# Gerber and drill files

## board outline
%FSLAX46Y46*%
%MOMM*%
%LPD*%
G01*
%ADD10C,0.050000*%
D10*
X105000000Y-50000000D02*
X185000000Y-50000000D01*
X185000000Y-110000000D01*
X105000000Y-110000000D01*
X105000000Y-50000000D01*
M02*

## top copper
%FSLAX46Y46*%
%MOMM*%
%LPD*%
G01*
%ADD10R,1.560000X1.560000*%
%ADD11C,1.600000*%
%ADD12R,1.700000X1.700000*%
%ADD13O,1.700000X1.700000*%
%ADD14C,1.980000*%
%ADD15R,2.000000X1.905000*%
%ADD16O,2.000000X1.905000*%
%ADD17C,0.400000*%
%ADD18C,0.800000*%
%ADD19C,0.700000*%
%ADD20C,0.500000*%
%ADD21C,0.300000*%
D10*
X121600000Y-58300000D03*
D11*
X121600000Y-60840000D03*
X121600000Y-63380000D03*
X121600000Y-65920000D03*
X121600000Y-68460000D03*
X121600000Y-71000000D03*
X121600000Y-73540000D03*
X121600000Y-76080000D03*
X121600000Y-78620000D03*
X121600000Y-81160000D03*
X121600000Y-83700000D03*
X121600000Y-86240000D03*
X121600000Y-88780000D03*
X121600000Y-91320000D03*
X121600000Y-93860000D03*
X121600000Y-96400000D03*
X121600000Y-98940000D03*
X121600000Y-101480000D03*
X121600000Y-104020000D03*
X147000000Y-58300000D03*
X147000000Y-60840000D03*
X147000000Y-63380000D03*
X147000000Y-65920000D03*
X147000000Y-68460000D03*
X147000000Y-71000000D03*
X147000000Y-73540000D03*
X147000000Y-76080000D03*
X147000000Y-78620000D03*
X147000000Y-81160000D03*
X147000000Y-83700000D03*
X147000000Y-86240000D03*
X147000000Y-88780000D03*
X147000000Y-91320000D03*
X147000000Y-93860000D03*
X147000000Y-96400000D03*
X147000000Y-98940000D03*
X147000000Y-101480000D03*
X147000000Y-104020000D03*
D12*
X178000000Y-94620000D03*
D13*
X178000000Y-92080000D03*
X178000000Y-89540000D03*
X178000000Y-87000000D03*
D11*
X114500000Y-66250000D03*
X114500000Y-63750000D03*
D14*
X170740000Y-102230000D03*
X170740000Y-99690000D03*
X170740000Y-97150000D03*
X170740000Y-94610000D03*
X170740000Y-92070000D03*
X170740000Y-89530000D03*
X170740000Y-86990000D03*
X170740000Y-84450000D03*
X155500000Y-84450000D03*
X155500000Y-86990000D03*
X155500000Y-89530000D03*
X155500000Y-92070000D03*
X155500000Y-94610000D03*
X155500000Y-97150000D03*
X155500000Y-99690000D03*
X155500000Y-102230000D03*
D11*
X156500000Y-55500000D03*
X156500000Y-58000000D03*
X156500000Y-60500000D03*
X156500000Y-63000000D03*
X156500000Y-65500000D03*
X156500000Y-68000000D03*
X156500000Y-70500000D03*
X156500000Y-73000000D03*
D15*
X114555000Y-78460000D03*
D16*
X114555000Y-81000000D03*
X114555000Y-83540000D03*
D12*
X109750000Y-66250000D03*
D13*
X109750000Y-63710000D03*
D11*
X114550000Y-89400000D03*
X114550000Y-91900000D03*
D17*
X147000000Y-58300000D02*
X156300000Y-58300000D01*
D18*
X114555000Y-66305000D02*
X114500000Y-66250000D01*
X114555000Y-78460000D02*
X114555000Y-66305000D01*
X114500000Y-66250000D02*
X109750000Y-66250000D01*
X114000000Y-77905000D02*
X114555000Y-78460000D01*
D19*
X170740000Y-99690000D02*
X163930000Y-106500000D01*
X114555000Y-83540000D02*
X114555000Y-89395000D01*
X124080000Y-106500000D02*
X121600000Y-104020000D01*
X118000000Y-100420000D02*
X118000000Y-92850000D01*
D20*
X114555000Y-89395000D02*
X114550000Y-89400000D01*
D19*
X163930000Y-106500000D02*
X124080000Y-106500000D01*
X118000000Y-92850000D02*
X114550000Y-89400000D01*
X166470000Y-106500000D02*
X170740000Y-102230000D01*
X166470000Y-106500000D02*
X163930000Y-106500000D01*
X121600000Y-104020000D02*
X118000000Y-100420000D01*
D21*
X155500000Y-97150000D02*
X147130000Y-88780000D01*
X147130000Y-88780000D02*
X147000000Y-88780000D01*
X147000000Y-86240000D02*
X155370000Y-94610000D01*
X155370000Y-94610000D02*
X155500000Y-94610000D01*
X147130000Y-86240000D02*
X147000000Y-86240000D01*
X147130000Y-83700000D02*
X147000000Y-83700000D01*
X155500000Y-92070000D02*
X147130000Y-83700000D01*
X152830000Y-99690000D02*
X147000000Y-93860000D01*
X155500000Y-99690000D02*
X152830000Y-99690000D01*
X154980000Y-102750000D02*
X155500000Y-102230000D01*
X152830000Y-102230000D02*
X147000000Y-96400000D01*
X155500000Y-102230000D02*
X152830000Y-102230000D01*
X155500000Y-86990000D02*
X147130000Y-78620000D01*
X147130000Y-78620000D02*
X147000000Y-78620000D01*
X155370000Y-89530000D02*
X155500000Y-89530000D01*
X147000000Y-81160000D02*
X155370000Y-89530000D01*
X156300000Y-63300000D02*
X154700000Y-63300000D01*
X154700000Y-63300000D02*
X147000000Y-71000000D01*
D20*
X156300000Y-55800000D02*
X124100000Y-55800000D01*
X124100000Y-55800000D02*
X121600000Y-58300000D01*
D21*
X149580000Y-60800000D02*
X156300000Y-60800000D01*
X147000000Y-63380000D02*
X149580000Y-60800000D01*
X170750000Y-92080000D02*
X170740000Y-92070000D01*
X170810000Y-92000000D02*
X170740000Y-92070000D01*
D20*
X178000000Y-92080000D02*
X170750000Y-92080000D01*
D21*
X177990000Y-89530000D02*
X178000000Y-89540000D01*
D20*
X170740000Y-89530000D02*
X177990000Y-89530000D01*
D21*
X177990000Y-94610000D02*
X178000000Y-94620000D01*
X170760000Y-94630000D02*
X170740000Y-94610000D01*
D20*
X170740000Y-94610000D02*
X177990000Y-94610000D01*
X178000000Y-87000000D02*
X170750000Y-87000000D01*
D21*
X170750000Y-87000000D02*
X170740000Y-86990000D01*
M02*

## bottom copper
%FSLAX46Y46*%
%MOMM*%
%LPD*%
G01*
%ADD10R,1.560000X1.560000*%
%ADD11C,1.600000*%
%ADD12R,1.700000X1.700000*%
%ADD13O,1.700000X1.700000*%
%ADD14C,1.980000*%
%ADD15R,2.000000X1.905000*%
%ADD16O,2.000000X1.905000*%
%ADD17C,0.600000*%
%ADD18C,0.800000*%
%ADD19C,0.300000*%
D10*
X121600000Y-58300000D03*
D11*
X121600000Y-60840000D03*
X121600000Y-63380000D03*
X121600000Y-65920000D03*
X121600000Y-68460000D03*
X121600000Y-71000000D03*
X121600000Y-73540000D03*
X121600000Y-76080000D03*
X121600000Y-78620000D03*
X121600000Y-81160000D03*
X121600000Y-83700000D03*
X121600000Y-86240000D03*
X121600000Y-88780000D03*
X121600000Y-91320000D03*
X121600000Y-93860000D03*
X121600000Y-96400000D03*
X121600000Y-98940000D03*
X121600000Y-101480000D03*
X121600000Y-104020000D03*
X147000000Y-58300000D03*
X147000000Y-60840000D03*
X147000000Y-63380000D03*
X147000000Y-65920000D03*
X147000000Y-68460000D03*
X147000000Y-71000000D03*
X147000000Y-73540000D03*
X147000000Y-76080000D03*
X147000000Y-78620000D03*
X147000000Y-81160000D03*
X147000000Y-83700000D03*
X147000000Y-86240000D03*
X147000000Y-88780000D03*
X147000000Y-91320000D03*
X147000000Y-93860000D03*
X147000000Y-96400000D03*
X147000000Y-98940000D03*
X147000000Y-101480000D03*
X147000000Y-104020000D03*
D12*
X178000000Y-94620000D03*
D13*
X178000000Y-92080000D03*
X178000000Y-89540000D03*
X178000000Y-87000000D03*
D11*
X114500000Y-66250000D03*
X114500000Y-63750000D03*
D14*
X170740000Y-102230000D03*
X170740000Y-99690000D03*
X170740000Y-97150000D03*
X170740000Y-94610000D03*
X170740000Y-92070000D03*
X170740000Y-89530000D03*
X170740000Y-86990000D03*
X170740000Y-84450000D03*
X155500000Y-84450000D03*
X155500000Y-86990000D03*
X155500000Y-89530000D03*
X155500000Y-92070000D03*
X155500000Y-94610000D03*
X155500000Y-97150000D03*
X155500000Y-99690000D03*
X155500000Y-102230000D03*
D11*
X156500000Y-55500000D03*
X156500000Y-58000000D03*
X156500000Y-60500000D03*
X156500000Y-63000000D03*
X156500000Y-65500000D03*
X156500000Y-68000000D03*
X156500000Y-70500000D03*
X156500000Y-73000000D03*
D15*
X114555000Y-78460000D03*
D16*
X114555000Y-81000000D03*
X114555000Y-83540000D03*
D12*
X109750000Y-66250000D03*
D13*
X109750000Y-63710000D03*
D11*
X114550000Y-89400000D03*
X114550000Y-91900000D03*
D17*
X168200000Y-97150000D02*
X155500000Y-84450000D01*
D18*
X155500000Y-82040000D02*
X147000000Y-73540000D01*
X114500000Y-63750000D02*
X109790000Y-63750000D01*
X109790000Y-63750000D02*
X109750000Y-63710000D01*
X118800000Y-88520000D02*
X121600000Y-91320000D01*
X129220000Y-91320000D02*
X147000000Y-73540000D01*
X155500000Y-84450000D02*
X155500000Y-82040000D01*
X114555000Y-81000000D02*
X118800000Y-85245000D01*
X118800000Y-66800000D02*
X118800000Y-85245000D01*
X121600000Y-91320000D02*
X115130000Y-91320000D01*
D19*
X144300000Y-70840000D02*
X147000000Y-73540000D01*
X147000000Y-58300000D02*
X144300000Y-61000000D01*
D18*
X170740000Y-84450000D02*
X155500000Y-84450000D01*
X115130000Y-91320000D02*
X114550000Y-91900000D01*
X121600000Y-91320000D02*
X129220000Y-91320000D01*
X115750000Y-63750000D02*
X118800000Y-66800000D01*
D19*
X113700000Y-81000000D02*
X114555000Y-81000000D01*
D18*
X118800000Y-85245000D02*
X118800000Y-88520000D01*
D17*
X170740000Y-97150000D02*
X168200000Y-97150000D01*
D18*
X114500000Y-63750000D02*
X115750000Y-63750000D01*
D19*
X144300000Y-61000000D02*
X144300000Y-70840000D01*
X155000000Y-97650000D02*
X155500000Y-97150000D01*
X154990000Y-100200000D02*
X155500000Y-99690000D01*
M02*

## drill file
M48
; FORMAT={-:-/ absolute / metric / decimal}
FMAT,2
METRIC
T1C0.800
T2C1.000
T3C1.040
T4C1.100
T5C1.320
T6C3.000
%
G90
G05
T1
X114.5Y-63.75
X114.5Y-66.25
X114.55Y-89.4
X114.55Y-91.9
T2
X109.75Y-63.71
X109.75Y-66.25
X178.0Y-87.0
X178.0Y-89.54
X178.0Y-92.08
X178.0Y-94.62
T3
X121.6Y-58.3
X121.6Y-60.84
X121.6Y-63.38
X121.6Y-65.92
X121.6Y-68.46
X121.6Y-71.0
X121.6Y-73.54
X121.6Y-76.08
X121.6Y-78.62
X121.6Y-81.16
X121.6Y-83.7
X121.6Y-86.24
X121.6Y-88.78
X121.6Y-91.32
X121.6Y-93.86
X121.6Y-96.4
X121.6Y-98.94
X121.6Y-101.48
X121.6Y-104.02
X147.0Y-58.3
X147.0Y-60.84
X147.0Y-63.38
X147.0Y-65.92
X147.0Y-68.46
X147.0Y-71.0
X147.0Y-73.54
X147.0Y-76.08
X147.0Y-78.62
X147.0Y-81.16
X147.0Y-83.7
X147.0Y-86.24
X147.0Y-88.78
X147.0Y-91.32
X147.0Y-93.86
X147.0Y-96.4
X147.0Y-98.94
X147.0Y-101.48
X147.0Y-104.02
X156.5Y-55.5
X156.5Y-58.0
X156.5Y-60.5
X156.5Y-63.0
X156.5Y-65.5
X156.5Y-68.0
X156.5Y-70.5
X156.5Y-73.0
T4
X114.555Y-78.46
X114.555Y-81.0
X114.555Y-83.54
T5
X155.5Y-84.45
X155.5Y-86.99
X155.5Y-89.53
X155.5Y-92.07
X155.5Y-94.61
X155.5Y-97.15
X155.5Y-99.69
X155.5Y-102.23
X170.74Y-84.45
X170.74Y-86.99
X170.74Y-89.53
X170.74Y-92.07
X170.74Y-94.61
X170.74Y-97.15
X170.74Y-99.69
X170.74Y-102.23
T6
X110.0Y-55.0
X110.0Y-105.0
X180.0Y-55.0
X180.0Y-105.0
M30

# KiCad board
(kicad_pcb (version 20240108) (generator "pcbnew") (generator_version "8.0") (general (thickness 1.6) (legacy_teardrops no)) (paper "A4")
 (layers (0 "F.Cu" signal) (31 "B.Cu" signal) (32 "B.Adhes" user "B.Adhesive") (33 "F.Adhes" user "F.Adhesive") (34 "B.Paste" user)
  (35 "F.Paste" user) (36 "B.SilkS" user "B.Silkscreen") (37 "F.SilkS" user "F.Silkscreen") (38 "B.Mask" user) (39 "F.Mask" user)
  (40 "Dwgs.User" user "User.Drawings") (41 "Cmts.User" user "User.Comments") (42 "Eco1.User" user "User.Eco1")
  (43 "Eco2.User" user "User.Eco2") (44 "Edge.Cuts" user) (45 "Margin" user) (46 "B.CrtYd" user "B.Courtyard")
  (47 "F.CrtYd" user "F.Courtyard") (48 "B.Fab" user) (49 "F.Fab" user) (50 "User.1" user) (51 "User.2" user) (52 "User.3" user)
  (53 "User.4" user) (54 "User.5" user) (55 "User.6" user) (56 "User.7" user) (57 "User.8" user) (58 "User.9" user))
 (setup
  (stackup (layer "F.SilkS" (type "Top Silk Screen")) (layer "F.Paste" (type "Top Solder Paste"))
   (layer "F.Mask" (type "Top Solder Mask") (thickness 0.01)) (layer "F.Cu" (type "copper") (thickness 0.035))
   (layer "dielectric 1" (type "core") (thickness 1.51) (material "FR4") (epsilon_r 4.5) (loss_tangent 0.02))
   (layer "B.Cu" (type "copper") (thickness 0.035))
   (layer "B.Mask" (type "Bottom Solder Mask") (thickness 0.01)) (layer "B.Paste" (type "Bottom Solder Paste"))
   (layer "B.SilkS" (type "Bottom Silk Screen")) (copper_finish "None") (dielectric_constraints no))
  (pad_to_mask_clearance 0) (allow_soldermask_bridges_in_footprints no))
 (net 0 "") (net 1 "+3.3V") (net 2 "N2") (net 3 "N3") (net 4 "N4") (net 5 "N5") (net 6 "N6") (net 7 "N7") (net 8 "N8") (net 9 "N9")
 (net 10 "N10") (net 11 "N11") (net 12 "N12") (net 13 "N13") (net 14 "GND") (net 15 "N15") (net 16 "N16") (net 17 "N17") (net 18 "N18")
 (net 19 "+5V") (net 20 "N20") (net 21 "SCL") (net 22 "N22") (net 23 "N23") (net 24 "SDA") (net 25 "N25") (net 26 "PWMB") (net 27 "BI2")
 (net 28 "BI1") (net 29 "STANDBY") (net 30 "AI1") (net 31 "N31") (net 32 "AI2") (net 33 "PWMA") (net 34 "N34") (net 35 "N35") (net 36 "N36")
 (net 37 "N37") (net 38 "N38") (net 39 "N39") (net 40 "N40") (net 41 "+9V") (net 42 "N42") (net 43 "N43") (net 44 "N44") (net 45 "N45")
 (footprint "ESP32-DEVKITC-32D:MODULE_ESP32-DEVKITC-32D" (layer "F.Cu") (at 134.3 78.06)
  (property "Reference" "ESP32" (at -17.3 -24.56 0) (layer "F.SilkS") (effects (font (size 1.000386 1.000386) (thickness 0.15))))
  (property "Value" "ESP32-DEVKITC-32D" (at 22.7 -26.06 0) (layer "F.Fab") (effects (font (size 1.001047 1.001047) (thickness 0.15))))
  (pad "J2-1" thru_hole rect (at -12.7 -19.76) (size 1.56 1.56) (drill 1.04) (layers "*.Cu" "*.Mask") (remove_unused_layers no)
   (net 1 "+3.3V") (solder_mask_margin 0.102))
  (pad "J2-2" thru_hole circle (at -12.7 -17.22) (size 1.6 1.6) (drill 1.04) (layers "*.Cu" "*.Mask") (remove_unused_layers no) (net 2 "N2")
   (solder_mask_margin 0.102))
  (pad "J2-3" thru_hole circle (at -12.7 -14.68) (size 1.6 1.6) (drill 1.04) (layers "*.Cu" "*.Mask") (remove_unused_layers no) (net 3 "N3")
   (solder_mask_margin 0.102))
  (pad "J2-4" thru_hole circle (at -12.7 -12.14) (size 1.6 1.6) (drill 1.04) (layers "*.Cu" "*.Mask") (remove_unused_layers no) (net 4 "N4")
   (solder_mask_margin 0.102))
  (pad "J2-5" thru_hole circle (at -12.7 -9.6) (size 1.6 1.6) (drill 1.04) (layers "*.Cu" "*.Mask") (remove_unused_layers no) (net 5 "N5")
   (solder_mask_margin 0.102))
  (pad "J2-6" thru_hole circle (at -12.7 -7.06) (size 1.6 1.6) (drill 1.04) (layers "*.Cu" "*.Mask") (remove_unused_layers no) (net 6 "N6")
   (solder_mask_margin 0.102))
  (pad "J2-7" thru_hole circle (at -12.7 -4.52) (size 1.6 1.6) (drill 1.04) (layers "*.Cu" "*.Mask") (remove_unused_layers no) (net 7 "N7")
   (solder_mask_margin 0.102))
  (pad "J2-8" thru_hole circle (at -12.7 -1.98) (size 1.6 1.6) (drill 1.04) (layers "*.Cu" "*.Mask") (remove_unused_layers no) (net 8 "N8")
   (solder_mask_margin 0.102))
  (pad "J2-9" thru_hole circle (at -12.7 0.56) (size 1.6 1.6) (drill 1.04) (layers "*.Cu" "*.Mask") (remove_unused_layers no) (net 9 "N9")
   (solder_mask_margin 0.102))
  (pad "J2-10" thru_hole circle (at -12.7 3.1) (size 1.6 1.6) (drill 1.04) (layers "*.Cu" "*.Mask") (remove_unused_layers no) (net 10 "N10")
   (solder_mask_margin 0.102))
  (pad "J2-11" thru_hole circle (at -12.7 5.64) (size 1.6 1.6) (drill 1.04) (layers "*.Cu" "*.Mask") (remove_unused_layers no)
   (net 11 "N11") (solder_mask_margin 0.102))
  (pad "J2-12" thru_hole circle (at -12.7 8.18) (size 1.6 1.6) (drill 1.04) (layers "*.Cu" "*.Mask") (remove_unused_layers no)
   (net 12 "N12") (solder_mask_margin 0.102))
  (pad "J2-13" thru_hole circle (at -12.7 10.72) (size 1.6 1.6) (drill 1.04) (layers "*.Cu" "*.Mask") (remove_unused_layers no)
   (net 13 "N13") (solder_mask_margin 0.102))
  (pad "J2-14" thru_hole circle (at -12.7 13.26) (size 1.6 1.6) (drill 1.04) (layers "*.Cu" "*.Mask") (remove_unused_layers no)
   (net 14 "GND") (solder_mask_margin 0.102))
  (pad "J2-15" thru_hole circle (at -12.7 15.8) (size 1.6 1.6) (drill 1.04) (layers "*.Cu" "*.Mask") (remove_unused_layers no)
   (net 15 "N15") (solder_mask_margin 0.102))
  (pad "J2-16" thru_hole circle (at -12.7 18.34) (size 1.6 1.6) (drill 1.04) (layers "*.Cu" "*.Mask") (remove_unused_layers no)
   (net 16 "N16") (solder_mask_margin 0.102))
  (pad "J2-17" thru_hole circle (at -12.7 20.88) (size 1.6 1.6) (drill 1.04) (layers "*.Cu" "*.Mask") (remove_unused_layers no)
   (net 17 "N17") (solder_mask_margin 0.102))
  (pad "J2-18" thru_hole circle (at -12.7 23.42) (size 1.6 1.6) (drill 1.04) (layers "*.Cu" "*.Mask") (remove_unused_layers no)
   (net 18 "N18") (solder_mask_margin 0.102))
  (pad "J2-19" thru_hole circle (at -12.7 25.96) (size 1.6 1.6) (drill 1.04) (layers "*.Cu" "*.Mask") (remove_unused_layers no)
   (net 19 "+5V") (solder_mask_margin 0.102))
  (pad "J3-1" thru_hole circle (at 12.7 -19.76) (size 1.6 1.6) (drill 1.04) (layers "*.Cu" "*.Mask") (remove_unused_layers no)
   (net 14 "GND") (solder_mask_margin 0.102))
  (pad "J3-2" thru_hole circle (at 12.7 -17.22) (size 1.6 1.6) (drill 1.04) (layers "*.Cu" "*.Mask") (remove_unused_layers no)
   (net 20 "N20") (solder_mask_margin 0.102))
  (pad "J3-3" thru_hole circle (at 12.7 -14.68) (size 1.6 1.6) (drill 1.04) (layers "*.Cu" "*.Mask") (remove_unused_layers no)
   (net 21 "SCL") (solder_mask_margin 0.102))
  (pad "J3-4" thru_hole circle (at 12.7 -12.14) (size 1.6 1.6) (drill 1.04) (layers "*.Cu" "*.Mask") (remove_unused_layers no)
   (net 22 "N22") (solder_mask_margin 0.102))
  (pad "J3-5" thru_hole circle (at 12.7 -9.6) (size 1.6 1.6) (drill 1.04) (layers "*.Cu" "*.Mask") (remove_unused_layers no) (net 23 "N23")
   (solder_mask_margin 0.102))
  (pad "J3-6" thru_hole circle (at 12.7 -7.06) (size 1.6 1.6) (drill 1.04) (layers "*.Cu" "*.Mask") (remove_unused_layers no) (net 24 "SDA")
   (solder_mask_margin 0.102))
  (pad "J3-7" thru_hole circle (at 12.7 -4.52) (size 1.6 1.6) (drill 1.04) (layers "*.Cu" "*.Mask") (remove_unused_layers no) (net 14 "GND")
   (solder_mask_margin 0.102))
  (pad "J3-8" thru_hole circle (at 12.7 -1.98) (size 1.6 1.6) (drill 1.04) (layers "*.Cu" "*.Mask") (remove_unused_layers no) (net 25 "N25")
   (solder_mask_margin 0.102))
  (pad "J3-9" thru_hole circle (at 12.7 0.56) (size 1.6 1.6) (drill 1.04) (layers "*.Cu" "*.Mask") (remove_unused_layers no) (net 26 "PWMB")
   (solder_mask_margin 0.102))
  (pad "J3-10" thru_hole circle (at 12.7 3.1) (size 1.6 1.6) (drill 1.04) (layers "*.Cu" "*.Mask") (remove_unused_layers no) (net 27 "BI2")
   (solder_mask_margin 0.102))
  (pad "J3-11" thru_hole circle (at 12.7 5.64) (size 1.6 1.6) (drill 1.04) (layers "*.Cu" "*.Mask") (remove_unused_layers no) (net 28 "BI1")
   (solder_mask_margin 0.102))
  (pad "J3-12" thru_hole circle (at 12.7 8.18) (size 1.6 1.6) (drill 1.04) (layers "*.Cu" "*.Mask") (remove_unused_layers no)
   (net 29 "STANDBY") (solder_mask_margin 0.102))
  (pad "J3-13" thru_hole circle (at 12.7 10.72) (size 1.6 1.6) (drill 1.04) (layers "*.Cu" "*.Mask") (remove_unused_layers no)
   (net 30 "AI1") (solder_mask_margin 0.102))
  (pad "J3-14" thru_hole circle (at 12.7 13.26) (size 1.6 1.6) (drill 1.04) (layers "*.Cu" "*.Mask") (remove_unused_layers no)
   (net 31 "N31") (solder_mask_margin 0.102))
  (pad "J3-15" thru_hole circle (at 12.7 15.8) (size 1.6 1.6) (drill 1.04) (layers "*.Cu" "*.Mask") (remove_unused_layers no) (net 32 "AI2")
   (solder_mask_margin 0.102))
  (pad "J3-16" thru_hole circle (at 12.7 18.34) (size 1.6 1.6) (drill 1.04) (layers "*.Cu" "*.Mask") (remove_unused_layers no)
   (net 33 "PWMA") (solder_mask_margin 0.102))
  (pad "J3-17" thru_hole circle (at 12.7 20.88) (size 1.6 1.6) (drill 1.04) (layers "*.Cu" "*.Mask") (remove_unused_layers no)
   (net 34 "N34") (solder_mask_margin 0.102))
  (pad "J3-18" thru_hole circle (at 12.7 23.42) (size 1.6 1.6) (drill 1.04) (layers "*.Cu" "*.Mask") (remove_unused_layers no)
   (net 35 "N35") (solder_mask_margin 0.102))
  (pad "J3-19" thru_hole circle (at 12.7 25.96) (size 1.6 1.6) (drill 1.04) (layers "*.Cu" "*.Mask") (remove_unused_layers no)
   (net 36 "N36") (solder_mask_margin 0.102)))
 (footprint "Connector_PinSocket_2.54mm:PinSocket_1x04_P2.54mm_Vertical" (layer "F.Cu") (at 178 94.62 180)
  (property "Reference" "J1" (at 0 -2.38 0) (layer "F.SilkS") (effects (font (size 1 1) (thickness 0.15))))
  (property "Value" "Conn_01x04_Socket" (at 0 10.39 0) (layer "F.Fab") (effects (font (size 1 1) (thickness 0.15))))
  (pad "1" thru_hole rect (at 0 0 180) (size 1.7 1.7) (drill 1) (layers "*.Cu" "*.Mask") (remove_unused_layers no) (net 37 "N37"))
  (pad "2" thru_hole oval (at 0 2.54 180) (size 1.7 1.7) (drill 1) (layers "*.Cu" "*.Mask") (remove_unused_layers no) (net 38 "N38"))
  (pad "3" thru_hole oval (at 0 5.08 180) (size 1.7 1.7) (drill 1) (layers "*.Cu" "*.Mask") (remove_unused_layers no) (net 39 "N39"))
  (pad "4" thru_hole oval (at 0 7.62 180) (size 1.7 1.7) (drill 1) (layers "*.Cu" "*.Mask") (remove_unused_layers no) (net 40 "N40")))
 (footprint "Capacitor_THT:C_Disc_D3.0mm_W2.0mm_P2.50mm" (layer "F.Cu") (at 114.5 66.25 90)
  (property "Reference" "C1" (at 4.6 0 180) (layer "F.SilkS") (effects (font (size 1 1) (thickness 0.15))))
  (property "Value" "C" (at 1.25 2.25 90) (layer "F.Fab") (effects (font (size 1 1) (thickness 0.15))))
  (pad "1" thru_hole circle (at 0 0 90) (size 1.6 1.6) (drill 0.8) (layers "*.Cu" "*.Mask") (remove_unused_layers no) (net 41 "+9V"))
  (pad "2" thru_hole circle (at 2.5 0 90) (size 1.6 1.6) (drill 0.8) (layers "*.Cu" "*.Mask") (remove_unused_layers no) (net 14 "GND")))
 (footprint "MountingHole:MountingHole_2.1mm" (layer "F.Cu") (at 180 55)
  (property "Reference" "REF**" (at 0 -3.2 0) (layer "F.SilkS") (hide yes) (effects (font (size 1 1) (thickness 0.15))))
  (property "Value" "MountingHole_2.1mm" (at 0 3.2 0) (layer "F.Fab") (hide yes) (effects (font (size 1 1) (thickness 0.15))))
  (pad "" np_thru_hole circle (at 0 0) (size 3 3) (drill 3) (layers "F&B.Cu" "*.Mask")))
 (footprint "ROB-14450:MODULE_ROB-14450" (layer "F.Cu") (at 163.12 93.34 180)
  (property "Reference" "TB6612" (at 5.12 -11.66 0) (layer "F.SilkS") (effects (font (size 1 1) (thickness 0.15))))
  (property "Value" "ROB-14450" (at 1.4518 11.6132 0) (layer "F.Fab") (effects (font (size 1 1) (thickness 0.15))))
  (pad "1" thru_hole circle (at -7.62 -8.89 180) (size 1.98 1.98) (drill 1.32) (layers "*.Cu" "*.Mask") (remove_unused_layers no)
   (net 19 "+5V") (solder_mask_margin 0.102))
  (pad "2" thru_hole circle (at -7.62 -6.35 180) (size 1.98 1.98) (drill 1.32) (layers "*.Cu" "*.Mask") (remove_unused_layers no)
   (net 19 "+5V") (solder_mask_margin 0.102))
  (pad "3" thru_hole circle (at -7.62 -3.81 180) (size 1.98 1.98) (drill 1.32) (layers "*.Cu" "*.Mask") (remove_unused_layers no)
   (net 14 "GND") (solder_mask_margin 0.102))
  (pad "4" thru_hole circle (at -7.62 -1.27 180) (size 1.98 1.98) (drill 1.32) (layers "*.Cu" "*.Mask") (remove_unused_layers no)
   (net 37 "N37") (solder_mask_margin 0.102))
  (pad "5" thru_hole circle (at -7.62 1.27 180) (size 1.98 1.98) (drill 1.32) (layers "*.Cu" "*.Mask") (remove_unused_layers no)
   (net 38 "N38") (solder_mask_margin 0.102))
  (pad "6" thru_hole circle (at -7.62 3.81 180) (size 1.98 1.98) (drill 1.32) (layers "*.Cu" "*.Mask") (remove_unused_layers no)
   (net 39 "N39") (solder_mask_margin 0.102))
  (pad "7" thru_hole circle (at -7.62 6.35 180) (size 1.98 1.98) (drill 1.32) (layers "*.Cu" "*.Mask") (remove_unused_layers no)
   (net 40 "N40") (solder_mask_margin 0.102))
  (pad "8" thru_hole circle (at -7.62 8.89 180) (size 1.98 1.98) (drill 1.32) (layers "*.Cu" "*.Mask") (remove_unused_layers no)
   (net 14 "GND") (solder_mask_margin 0.102))
  (pad "9" thru_hole circle (at 7.62 8.89 180) (size 1.98 1.98) (drill 1.32) (layers "*.Cu" "*.Mask") (remove_unused_layers no)
   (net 14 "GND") (solder_mask_margin 0.102))
  (pad "10" thru_hole circle (at 7.62 6.35 180) (size 1.98 1.98) (drill 1.32) (layers "*.Cu" "*.Mask") (remove_unused_layers no)
   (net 26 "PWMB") (solder_mask_margin 0.102))
  (pad "11" thru_hole circle (at 7.62 3.81 180) (size 1.98 1.98) (drill 1.32) (layers "*.Cu" "*.Mask") (remove_unused_layers no)
   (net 27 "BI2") (solder_mask_margin 0.102))
  (pad "12" thru_hole circle (at 7.62 1.27 180) (size 1.98 1.98) (drill 1.32) (layers "*.Cu" "*.Mask") (remove_unused_layers no)
   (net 28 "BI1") (solder_mask_margin 0.102))
  (pad "13" thru_hole circle (at 7.62 -1.27 180) (size 1.98 1.98) (drill 1.32) (layers "*.Cu" "*.Mask") (remove_unused_layers no)
   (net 29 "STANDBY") (solder_mask_margin 0.102))
  (pad "14" thru_hole circle (at 7.62 -3.81 180) (size 1.98 1.98) (drill 1.32) (layers "*.Cu" "*.Mask") (remove_unused_layers no)
   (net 30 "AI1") (solder_mask_margin 0.102))
  (pad "15" thru_hole circle (at 7.62 -6.35 180) (size 1.98 1.98) (drill 1.32) (layers "*.Cu" "*.Mask") (remove_unused_layers no)
   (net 32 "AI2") (solder_mask_margin 0.102))
  (pad "16" thru_hole circle (at 7.62 -8.89 180) (size 1.98 1.98) (drill 1.32) (layers "*.Cu" "*.Mask") (remove_unused_layers no)
   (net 33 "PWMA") (solder_mask_margin 0.102)))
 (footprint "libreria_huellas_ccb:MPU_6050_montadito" (layer "F.Cu") (at 155 75.2)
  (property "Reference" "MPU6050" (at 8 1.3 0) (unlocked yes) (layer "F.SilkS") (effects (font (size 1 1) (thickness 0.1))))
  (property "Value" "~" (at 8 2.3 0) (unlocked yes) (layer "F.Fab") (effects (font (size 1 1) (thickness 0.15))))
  (pad "1" thru_hole circle (at 1.5 -19.7) (size 1.6 1.6) (drill 1.04) (layers "*.Cu" "*.Mask") (remove_unused_layers no) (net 1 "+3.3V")
   (solder_mask_margin 0.102))
  (pad "2" thru_hole circle (at 1.5 -17.2) (size 1.6 1.6) (drill 1.04) (layers "*.Cu" "*.Mask") (remove_unused_layers no) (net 14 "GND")
   (solder_mask_margin 0.102))
  (pad "3" thru_hole circle (at 1.5 -14.7) (size 1.6 1.6) (drill 1.04) (layers "*.Cu" "*.Mask") (remove_unused_layers no) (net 21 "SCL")
   (solder_mask_margin 0.102))
  (pad "4" thru_hole circle (at 1.5 -12.2) (size 1.6 1.6) (drill 1.04) (layers "*.Cu" "*.Mask") (remove_unused_layers no) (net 24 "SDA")
   (solder_mask_margin 0.102))
  (pad "5" thru_hole circle (at 1.5 -9.7) (size 1.6 1.6) (drill 1.04) (layers "*.Cu" "*.Mask") (remove_unused_layers no) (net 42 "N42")
   (solder_mask_margin 0.102))
  (pad "6" thru_hole circle (at 1.5 -7.2) (size 1.6 1.6) (drill 1.04) (layers "*.Cu" "*.Mask") (remove_unused_layers no) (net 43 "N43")
   (solder_mask_margin 0.102))
  (pad "7" thru_hole circle (at 1.5 -4.7) (size 1.6 1.6) (drill 1.04) (layers "*.Cu" "*.Mask") (remove_unused_layers no) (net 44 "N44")
   (solder_mask_margin 0.102))
  (pad "8" thru_hole circle (at 1.5 -2.2) (size 1.6 1.6) (drill 1.04) (layers "*.Cu" "*.Mask") (remove_unused_layers no) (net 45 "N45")
   (solder_mask_margin 0.102)))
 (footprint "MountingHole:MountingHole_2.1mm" (layer "F.Cu") (at 110 55)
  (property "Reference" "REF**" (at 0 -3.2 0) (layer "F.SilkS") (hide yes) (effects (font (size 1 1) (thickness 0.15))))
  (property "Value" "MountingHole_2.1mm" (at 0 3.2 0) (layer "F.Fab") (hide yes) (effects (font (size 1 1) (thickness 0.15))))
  (pad "" np_thru_hole circle (at 0 0) (size 3 3) (drill 3) (layers "F&B.Cu" "*.Mask")))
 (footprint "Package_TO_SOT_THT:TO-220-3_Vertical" (layer "F.Cu") (at 114.555 78.46 -90)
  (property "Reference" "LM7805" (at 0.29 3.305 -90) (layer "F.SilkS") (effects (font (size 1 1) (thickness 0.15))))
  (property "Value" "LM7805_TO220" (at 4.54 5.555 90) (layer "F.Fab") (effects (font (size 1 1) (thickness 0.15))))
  (pad "1" thru_hole rect (at 0 0 270) (size 1.905 2) (drill 1.1) (layers "*.Cu" "*.Mask") (remove_unused_layers no) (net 41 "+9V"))
  (pad "2" thru_hole oval (at 2.54 0 270) (size 1.905 2) (drill 1.1) (layers "*.Cu" "*.Mask") (remove_unused_layers no) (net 14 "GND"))
  (pad "3" thru_hole oval (at 5.08 0 270) (size 1.905 2) (drill 1.1) (layers "*.Cu" "*.Mask") (remove_unused_layers no) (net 19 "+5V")))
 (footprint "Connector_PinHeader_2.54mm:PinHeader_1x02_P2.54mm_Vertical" (layer "F.Cu") (at 109.75 66.25 180)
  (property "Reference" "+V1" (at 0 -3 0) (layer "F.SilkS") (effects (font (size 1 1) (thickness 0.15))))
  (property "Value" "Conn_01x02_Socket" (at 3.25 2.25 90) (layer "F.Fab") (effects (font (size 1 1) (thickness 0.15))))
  (pad "1" thru_hole rect (at 0 0 180) (size 1.7 1.7) (drill 1) (layers "*.Cu" "*.Mask") (remove_unused_layers no) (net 41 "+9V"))
  (pad "2" thru_hole oval (at 0 2.54 180) (size 1.7 1.7) (drill 1) (layers "*.Cu" "*.Mask") (remove_unused_layers no) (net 14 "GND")))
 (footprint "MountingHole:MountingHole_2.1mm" (layer "F.Cu") (at 180 105)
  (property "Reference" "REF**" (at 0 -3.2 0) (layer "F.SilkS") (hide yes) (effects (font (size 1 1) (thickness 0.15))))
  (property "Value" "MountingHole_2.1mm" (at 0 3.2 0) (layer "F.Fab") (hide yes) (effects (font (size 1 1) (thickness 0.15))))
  (pad "" np_thru_hole circle (at 0 0) (size 3 3) (drill 3) (layers "F&B.Cu" "*.Mask")))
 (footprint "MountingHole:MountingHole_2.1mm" (layer "F.Cu") (at 110 105)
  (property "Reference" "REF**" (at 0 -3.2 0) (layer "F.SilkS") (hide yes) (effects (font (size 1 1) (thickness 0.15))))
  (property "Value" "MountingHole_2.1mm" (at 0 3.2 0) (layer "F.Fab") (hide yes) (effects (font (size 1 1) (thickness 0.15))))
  (pad "" np_thru_hole circle (at 0 0) (size 3 3) (drill 3) (layers "F&B.Cu" "*.Mask")))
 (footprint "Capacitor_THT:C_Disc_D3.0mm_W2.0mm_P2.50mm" (layer "F.Cu") (at 114.55 89.4 -90)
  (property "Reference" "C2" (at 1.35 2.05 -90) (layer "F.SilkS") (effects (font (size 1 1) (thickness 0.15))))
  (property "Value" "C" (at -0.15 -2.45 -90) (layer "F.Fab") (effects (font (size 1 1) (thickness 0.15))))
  (pad "1" thru_hole circle (at 0 0 270) (size 1.6 1.6) (drill 0.8) (layers "*.Cu" "*.Mask") (remove_unused_layers no) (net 19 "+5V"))
  (pad "2" thru_hole circle (at 2.5 0 270) (size 1.6 1.6) (drill 0.8) (layers "*.Cu" "*.Mask") (remove_unused_layers no) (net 14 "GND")))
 (gr_rect (start 105 50) (end 185 110) (stroke (width 0.05) (type default)) (fill none) (layer "Edge.Cuts"))
 (segment (start 147 58.3) (end 156.3 58.3) (width 0.4) (layer "F.Cu") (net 14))
 (segment (start 168.2 97.15) (end 155.5 84.45) (width 0.6) (layer "B.Cu") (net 14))
 (segment (start 155.5 82.04) (end 147 73.54) (width 0.8) (layer "B.Cu") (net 14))
 (segment (start 114.5 63.75) (end 109.79 63.75) (width 0.8) (layer "B.Cu") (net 14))
 (segment (start 109.79 63.75) (end 109.75 63.71) (width 0.8) (layer "B.Cu") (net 14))
 (segment (start 118.8 88.52) (end 121.6 91.32) (width 0.8) (layer "B.Cu") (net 14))
 (segment (start 129.22 91.32) (end 147 73.54) (width 0.8) (layer "B.Cu") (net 14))
 (segment (start 155.5 84.45) (end 155.5 82.04) (width 0.8) (layer "B.Cu") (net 14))
 (segment (start 114.555 81) (end 118.8 85.245) (width 0.8) (layer "B.Cu") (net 14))
 (segment (start 118.8 66.8) (end 118.8 85.245) (width 0.8) (layer "B.Cu") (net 14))
 (segment (start 121.6 91.32) (end 115.13 91.32) (width 0.8) (layer "B.Cu") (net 14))
 (segment (start 144.3 70.84) (end 147 73.54) (width 0.3) (layer "B.Cu") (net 14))
 (segment (start 147 58.3) (end 144.3 61) (width 0.3) (layer "B.Cu") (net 14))
 (segment (start 170.74 84.45) (end 155.5 84.45) (width 0.8) (layer "B.Cu") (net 14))
 (segment (start 115.13 91.32) (end 114.55 91.9) (width 0.8) (layer "B.Cu") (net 14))
 (segment (start 121.6 91.32) (end 129.22 91.32) (width 0.8) (layer "B.Cu") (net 14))
 (segment (start 115.75 63.75) (end 118.8 66.8) (width 0.8) (layer "B.Cu") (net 14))
 (segment (start 113.7 81) (end 114.555 81) (width 0.3) (layer "B.Cu") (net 14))
 (segment (start 118.8 85.245) (end 118.8 88.52) (width 0.8) (layer "B.Cu") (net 14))
 (segment (start 170.74 97.15) (end 168.2 97.15) (width 0.6) (layer "B.Cu") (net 14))
 (segment (start 114.5 63.75) (end 115.75 63.75) (width 0.8) (layer "B.Cu") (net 14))
 (segment (start 144.3 61) (end 144.3 70.84) (width 0.3) (layer "B.Cu") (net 14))
 (segment (start 114.555 66.305) (end 114.5 66.25) (width 0.8) (layer "F.Cu") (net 41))
 (segment (start 114.555 78.46) (end 114.555 66.305) (width 0.8) (layer "F.Cu") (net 41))
 (segment (start 114.5 66.25) (end 109.75 66.25) (width 0.8) (layer "F.Cu") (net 41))
 (segment (start 114 77.905) (end 114.555 78.46) (width 0.8) (layer "F.Cu") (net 41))
 (segment (start 170.74 99.69) (end 163.93 106.5) (width 0.7) (layer "F.Cu") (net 19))
 (segment (start 114.555 83.54) (end 114.555 89.395) (width 0.7) (layer "F.Cu") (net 19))
 (segment (start 124.08 106.5) (end 121.6 104.02) (width 0.7) (layer "F.Cu") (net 19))
 (segment (start 118 100.42) (end 118 92.85) (width 0.7) (layer "F.Cu") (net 19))
 (segment (start 114.555 89.395) (end 114.55 89.4) (width 0.5) (layer "F.Cu") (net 19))
 (segment (start 163.93 106.5) (end 124.08 106.5) (width 0.7) (layer "F.Cu") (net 19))
 (segment (start 118 92.85) (end 114.55 89.4) (width 0.7) (layer "F.Cu") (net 19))
 (segment (start 166.47 106.5) (end 170.74 102.23) (width 0.7) (layer "F.Cu") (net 19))
 (segment (start 166.47 106.5) (end 163.93 106.5) (width 0.7) (layer "F.Cu") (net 19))
 (segment (start 121.6 104.02) (end 118 100.42) (width 0.7) (layer "F.Cu") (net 19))
 (segment (start 155.5 97.15) (end 147.13 88.78) (width 0.3) (layer "F.Cu") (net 30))
 (segment (start 147.13 88.78) (end 147 88.78) (width 0.3) (layer "F.Cu") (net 30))
 (segment (start 155 97.65) (end 155.5 97.15) (width 0.3) (layer "B.Cu") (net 30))
 (segment (start 147 86.24) (end 155.37 94.61) (width 0.3) (layer "F.Cu") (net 29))
 (segment (start 155.37 94.61) (end 155.5 94.61) (width 0.3) (layer "F.Cu") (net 29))
 (segment (start 147.13 86.24) (end 147 86.24) (width 0.3) (layer "F.Cu") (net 29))
 (segment (start 147.13 83.7) (end 147 83.7) (width 0.3) (layer "F.Cu") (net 28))
 (segment (start 155.5 92.07) (end 147.13 83.7) (width 0.3) (layer "F.Cu") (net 28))
 (segment (start 152.83 99.69) (end 147 93.86) (width 0.3) (layer "F.Cu") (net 32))
 (segment (start 155.5 99.69) (end 152.83 99.69) (width 0.3) (layer "F.Cu") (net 32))
 (segment (start 154.99 100.2) (end 155.5 99.69) (width 0.3) (layer "B.Cu") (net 32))
 (segment (start 154.98 102.75) (end 155.5 102.23) (width 0.3) (layer "F.Cu") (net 33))
 (segment (start 152.83 102.23) (end 147 96.4) (width 0.3) (layer "F.Cu") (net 33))
 (segment (start 155.5 102.23) (end 152.83 102.23) (width 0.3) (layer "F.Cu") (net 33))
 (segment (start 155.5 86.99) (end 147.13 78.62) (width 0.3) (layer "F.Cu") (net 26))
 (segment (start 147.13 78.62) (end 147 78.62) (width 0.3) (layer "F.Cu") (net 26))
 (segment (start 155.37 89.53) (end 155.5 89.53) (width 0.3) (layer "F.Cu") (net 27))
 (segment (start 147 81.16) (end 155.37 89.53) (width 0.3) (layer "F.Cu") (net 27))
 (segment (start 156.3 63.3) (end 154.7 63.3) (width 0.3) (layer "F.Cu") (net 24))
 (segment (start 154.7 63.3) (end 147 71) (width 0.3) (layer "F.Cu") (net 24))
 (segment (start 156.3 55.8) (end 124.1 55.8) (width 0.5) (layer "F.Cu") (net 1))
 (segment (start 124.1 55.8) (end 121.6 58.3) (width 0.5) (layer "F.Cu") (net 1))
 (segment (start 149.58 60.8) (end 156.3 60.8) (width 0.3) (layer "F.Cu") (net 21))
 (segment (start 147 63.38) (end 149.58 60.8) (width 0.3) (layer "F.Cu") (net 21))
 (segment (start 170.75 92.08) (end 170.74 92.07) (width 0.3) (layer "F.Cu") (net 38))
 (segment (start 170.81 92) (end 170.74 92.07) (width 0.3) (layer "F.Cu") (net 38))
 (segment (start 178 92.08) (end 170.75 92.08) (width 0.5) (layer "F.Cu") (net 38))
 (segment (start 177.99 89.53) (end 178 89.54) (width 0.3) (layer "F.Cu") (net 39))
 (segment (start 170.74 89.53) (end 177.99 89.53) (width 0.5) (layer "F.Cu") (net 39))
 (segment (start 177.99 94.61) (end 178 94.62) (width 0.3) (layer "F.Cu") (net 37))
 (segment (start 170.76 94.63) (end 170.74 94.61) (width 0.3) (layer "F.Cu") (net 37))
 (segment (start 170.74 94.61) (end 177.99 94.61) (width 0.5) (layer "F.Cu") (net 37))
 (segment (start 178 87) (end 170.75 87) (width 0.5) (layer "F.Cu") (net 40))
 (segment (start 170.75 87) (end 170.74 86.99) (width 0.3) (layer "F.Cu") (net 40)))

